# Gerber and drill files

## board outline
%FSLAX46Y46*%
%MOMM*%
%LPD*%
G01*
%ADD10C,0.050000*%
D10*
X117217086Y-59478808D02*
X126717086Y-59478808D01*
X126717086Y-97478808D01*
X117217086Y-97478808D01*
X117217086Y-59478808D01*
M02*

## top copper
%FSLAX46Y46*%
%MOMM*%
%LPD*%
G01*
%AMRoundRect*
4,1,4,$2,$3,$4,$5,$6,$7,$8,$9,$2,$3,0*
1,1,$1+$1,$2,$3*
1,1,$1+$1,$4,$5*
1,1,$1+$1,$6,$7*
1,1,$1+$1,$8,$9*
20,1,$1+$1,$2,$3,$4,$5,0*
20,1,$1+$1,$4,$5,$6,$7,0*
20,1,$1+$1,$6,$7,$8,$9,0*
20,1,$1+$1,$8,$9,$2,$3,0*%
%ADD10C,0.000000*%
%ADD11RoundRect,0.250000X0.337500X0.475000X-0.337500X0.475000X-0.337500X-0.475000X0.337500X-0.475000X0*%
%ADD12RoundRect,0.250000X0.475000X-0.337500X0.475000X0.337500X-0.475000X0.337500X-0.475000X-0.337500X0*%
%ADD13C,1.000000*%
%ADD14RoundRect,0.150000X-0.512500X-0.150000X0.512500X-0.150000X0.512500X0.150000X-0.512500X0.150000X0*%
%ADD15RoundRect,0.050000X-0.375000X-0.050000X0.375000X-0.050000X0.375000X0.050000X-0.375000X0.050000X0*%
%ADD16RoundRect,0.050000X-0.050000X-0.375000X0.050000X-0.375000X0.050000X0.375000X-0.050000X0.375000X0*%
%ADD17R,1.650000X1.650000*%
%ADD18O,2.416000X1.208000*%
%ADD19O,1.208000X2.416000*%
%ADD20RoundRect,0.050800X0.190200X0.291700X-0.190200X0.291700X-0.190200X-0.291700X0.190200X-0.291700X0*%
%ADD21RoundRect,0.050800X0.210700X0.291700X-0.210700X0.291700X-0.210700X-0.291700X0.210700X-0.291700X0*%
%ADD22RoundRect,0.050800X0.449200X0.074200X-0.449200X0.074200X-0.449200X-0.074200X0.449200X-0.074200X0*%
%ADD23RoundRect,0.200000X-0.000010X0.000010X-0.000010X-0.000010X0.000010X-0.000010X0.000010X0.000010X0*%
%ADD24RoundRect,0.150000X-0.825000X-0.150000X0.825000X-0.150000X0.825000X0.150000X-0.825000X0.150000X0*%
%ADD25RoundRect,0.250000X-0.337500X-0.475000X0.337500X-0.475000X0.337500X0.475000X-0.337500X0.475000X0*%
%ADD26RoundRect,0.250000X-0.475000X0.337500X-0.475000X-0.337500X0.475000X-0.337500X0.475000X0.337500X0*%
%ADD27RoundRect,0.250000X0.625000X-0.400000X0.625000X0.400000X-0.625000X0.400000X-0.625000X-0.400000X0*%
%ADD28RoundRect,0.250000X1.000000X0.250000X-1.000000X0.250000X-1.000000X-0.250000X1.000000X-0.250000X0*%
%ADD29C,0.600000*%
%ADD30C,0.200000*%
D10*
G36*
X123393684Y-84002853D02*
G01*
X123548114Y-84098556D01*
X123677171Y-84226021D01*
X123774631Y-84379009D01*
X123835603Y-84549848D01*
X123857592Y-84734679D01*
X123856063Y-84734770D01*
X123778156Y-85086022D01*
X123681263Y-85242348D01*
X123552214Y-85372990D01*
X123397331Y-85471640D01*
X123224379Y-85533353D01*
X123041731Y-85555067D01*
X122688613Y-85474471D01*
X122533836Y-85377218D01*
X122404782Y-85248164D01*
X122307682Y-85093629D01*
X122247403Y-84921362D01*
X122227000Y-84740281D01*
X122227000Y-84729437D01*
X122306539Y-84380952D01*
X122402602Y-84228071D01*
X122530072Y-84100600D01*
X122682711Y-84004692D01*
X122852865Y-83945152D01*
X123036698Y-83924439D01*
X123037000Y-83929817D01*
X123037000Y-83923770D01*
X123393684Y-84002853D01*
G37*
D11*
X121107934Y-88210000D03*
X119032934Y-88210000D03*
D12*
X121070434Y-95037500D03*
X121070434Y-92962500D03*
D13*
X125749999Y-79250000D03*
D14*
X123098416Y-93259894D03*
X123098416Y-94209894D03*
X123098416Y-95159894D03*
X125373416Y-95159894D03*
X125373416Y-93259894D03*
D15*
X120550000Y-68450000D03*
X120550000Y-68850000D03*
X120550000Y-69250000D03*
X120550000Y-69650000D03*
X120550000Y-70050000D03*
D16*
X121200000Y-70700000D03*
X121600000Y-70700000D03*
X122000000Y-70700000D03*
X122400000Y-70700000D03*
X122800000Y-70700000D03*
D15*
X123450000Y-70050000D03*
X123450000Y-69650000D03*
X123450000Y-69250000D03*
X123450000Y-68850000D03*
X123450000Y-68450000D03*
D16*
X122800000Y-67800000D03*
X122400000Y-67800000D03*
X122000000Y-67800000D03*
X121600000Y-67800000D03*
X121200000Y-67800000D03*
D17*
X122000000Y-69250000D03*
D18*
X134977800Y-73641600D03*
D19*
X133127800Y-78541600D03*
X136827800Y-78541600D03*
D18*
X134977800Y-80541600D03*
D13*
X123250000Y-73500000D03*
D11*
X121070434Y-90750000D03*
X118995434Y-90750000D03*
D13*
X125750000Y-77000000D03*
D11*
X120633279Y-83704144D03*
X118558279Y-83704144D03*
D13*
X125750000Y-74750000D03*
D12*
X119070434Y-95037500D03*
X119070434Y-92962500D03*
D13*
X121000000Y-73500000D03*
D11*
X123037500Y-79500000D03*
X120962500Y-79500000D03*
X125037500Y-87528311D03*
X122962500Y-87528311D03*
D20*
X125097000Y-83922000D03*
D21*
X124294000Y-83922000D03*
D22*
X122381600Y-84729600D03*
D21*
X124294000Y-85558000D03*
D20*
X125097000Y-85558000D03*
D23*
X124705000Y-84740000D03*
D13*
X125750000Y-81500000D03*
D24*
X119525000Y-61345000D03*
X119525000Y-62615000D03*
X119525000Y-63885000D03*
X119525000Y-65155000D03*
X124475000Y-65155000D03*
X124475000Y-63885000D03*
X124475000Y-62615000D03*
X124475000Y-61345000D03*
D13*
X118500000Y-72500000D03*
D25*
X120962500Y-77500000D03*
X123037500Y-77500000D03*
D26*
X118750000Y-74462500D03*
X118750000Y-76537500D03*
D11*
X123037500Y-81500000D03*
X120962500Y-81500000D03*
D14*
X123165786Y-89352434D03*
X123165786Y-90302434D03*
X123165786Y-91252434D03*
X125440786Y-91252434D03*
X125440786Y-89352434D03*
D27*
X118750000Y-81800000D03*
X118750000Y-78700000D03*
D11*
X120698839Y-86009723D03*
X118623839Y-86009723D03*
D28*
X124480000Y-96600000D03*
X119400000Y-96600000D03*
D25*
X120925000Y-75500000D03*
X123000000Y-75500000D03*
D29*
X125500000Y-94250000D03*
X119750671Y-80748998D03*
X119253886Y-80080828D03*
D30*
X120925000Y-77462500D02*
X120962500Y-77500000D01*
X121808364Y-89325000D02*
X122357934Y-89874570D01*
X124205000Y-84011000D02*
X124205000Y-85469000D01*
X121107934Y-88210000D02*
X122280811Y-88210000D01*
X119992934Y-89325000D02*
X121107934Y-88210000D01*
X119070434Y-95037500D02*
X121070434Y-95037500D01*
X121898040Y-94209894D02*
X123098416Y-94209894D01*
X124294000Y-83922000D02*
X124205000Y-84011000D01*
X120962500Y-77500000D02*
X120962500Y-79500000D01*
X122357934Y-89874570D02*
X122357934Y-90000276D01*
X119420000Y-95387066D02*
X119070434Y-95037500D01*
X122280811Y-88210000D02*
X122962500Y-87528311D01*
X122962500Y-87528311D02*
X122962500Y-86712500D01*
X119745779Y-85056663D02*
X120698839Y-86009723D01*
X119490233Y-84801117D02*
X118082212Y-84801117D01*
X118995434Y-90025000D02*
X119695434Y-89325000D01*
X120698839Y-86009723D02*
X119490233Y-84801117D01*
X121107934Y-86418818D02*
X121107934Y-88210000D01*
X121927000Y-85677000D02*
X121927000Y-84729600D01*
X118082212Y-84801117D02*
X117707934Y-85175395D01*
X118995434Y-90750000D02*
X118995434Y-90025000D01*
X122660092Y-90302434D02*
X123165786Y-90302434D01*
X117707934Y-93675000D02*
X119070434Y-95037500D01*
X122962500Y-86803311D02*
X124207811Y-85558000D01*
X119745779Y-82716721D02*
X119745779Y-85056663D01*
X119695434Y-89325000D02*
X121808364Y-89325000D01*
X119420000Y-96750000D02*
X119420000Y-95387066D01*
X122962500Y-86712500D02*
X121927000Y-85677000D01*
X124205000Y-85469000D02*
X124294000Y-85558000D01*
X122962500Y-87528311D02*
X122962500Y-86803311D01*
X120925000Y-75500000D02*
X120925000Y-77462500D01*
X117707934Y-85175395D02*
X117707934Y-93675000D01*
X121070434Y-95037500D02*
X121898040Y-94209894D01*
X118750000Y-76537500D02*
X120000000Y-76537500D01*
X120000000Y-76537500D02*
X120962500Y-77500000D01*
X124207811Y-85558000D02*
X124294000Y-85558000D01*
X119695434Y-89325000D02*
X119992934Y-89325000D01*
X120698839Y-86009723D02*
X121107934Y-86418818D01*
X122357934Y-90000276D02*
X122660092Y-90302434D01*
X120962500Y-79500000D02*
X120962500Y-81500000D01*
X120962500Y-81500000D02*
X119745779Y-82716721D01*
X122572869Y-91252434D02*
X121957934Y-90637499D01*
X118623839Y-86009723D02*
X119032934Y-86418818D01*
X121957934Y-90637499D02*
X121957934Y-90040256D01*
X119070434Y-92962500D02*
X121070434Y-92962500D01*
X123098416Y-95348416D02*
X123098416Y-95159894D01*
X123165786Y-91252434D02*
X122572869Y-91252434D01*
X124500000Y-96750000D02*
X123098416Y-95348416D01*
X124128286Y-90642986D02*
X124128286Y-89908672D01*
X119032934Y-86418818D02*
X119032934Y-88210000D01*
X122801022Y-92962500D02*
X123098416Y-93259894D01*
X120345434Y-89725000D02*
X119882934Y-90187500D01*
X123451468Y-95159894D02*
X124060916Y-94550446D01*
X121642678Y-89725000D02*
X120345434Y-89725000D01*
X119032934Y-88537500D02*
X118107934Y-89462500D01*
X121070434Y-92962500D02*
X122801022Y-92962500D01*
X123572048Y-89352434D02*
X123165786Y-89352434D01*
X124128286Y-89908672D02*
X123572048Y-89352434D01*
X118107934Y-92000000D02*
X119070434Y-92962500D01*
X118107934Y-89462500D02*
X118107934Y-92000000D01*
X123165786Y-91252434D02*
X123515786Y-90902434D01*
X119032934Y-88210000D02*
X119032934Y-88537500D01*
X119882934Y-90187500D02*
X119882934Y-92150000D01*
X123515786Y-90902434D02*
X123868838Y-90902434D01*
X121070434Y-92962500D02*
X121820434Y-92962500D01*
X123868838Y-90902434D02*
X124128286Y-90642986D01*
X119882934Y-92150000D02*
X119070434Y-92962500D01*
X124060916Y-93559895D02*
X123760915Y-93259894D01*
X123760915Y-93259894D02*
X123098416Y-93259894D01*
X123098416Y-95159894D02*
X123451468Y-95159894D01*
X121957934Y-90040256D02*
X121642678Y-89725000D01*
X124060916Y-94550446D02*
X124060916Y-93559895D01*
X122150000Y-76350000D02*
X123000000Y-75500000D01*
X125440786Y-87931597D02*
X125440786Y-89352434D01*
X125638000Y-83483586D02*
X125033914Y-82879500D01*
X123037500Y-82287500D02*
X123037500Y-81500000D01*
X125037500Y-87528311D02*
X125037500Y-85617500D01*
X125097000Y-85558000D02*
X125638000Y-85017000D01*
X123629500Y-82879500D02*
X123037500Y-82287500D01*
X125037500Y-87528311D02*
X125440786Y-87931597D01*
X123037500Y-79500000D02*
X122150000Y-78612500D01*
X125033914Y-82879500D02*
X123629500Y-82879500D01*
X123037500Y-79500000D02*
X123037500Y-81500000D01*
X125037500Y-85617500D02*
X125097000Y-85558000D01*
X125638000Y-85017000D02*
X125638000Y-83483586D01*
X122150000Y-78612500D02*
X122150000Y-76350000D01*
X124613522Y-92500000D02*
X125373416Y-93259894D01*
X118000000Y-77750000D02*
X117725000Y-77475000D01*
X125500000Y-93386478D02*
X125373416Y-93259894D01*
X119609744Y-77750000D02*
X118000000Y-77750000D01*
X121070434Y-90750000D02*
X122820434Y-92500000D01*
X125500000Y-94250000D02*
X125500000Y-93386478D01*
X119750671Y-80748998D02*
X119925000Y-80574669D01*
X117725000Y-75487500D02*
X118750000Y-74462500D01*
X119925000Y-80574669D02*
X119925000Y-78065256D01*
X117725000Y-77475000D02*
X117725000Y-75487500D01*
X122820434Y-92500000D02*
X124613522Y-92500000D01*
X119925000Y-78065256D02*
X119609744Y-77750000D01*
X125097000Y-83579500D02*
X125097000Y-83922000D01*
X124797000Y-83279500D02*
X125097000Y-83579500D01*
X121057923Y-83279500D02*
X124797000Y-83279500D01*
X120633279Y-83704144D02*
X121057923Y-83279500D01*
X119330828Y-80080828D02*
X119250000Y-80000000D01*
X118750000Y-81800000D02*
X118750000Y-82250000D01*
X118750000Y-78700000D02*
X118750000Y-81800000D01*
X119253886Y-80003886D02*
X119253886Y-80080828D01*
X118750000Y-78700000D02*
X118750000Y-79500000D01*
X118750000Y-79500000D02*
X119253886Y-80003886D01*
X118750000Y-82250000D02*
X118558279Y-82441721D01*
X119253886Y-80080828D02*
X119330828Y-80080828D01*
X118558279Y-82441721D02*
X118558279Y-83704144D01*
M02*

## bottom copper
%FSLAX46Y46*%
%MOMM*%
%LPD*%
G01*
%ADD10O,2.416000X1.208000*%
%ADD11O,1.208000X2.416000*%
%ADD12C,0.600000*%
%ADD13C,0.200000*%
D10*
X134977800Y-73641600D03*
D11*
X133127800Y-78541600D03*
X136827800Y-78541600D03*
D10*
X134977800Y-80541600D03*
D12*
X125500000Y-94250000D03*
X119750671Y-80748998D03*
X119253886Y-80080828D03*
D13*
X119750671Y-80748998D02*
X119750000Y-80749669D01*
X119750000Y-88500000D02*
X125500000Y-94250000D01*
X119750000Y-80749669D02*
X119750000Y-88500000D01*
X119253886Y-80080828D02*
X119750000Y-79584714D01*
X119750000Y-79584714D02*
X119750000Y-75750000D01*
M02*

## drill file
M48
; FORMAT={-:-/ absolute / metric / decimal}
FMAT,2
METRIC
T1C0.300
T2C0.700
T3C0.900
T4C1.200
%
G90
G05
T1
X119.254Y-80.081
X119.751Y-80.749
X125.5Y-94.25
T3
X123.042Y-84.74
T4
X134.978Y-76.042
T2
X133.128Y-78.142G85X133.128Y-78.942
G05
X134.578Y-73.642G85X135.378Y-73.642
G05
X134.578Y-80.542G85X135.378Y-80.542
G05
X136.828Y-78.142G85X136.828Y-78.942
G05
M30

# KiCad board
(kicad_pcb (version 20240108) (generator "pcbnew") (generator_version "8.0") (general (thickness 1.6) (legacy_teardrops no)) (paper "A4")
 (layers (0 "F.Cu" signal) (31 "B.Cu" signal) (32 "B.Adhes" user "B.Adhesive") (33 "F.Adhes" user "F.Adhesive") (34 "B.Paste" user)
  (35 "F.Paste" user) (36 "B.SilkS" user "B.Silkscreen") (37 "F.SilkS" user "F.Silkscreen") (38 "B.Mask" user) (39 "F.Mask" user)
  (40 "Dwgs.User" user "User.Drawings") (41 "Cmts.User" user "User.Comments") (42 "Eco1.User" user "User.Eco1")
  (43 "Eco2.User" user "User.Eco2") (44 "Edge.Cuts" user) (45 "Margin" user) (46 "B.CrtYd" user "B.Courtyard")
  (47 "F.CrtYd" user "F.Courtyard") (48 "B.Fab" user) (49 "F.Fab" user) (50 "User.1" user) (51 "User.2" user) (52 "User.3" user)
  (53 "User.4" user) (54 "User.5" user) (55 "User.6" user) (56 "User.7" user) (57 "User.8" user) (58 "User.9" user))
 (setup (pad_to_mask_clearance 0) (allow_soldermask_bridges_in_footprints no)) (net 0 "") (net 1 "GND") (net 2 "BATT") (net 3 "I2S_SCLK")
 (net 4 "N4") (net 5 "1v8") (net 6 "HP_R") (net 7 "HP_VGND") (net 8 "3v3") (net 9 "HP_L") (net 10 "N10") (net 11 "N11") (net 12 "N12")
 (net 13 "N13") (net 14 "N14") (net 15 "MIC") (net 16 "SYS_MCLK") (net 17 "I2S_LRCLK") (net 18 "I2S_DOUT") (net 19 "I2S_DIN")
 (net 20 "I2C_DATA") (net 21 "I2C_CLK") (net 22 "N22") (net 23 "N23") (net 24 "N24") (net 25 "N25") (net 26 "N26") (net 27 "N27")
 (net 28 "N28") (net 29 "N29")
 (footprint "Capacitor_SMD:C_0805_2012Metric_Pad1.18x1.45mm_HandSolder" (layer "F.Cu") (at 120.070434 88.21 180)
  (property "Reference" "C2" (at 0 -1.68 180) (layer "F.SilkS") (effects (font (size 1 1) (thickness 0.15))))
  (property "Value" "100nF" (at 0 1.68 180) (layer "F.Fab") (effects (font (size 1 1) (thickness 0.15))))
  (pad "1" smd roundrect (at -1.0375 0 180) (size 1.175 1.45) (layers "F.Cu" "F.Paste" "F.Mask") (roundrect_rratio 0.212766) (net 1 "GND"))
  (pad "2" smd roundrect (at 1.0375 0 180) (size 1.175 1.45) (layers "F.Cu" "F.Paste" "F.Mask") (roundrect_rratio 0.212766) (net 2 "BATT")))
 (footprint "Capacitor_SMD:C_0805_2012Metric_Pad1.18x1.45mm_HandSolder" (layer "F.Cu") (at 121.070434 94 90)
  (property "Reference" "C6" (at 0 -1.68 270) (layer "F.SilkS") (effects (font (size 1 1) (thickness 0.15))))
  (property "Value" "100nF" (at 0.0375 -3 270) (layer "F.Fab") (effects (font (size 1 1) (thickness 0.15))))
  (pad "1" smd roundrect (at -1.0375 0 90) (size 1.175 1.45) (layers "F.Cu" "F.Paste" "F.Mask") (roundrect_rratio 0.212766) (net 1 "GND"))
  (pad "2" smd roundrect (at 1.0375 0 90) (size 1.175 1.45) (layers "F.Cu" "F.Paste" "F.Mask") (roundrect_rratio 0.212766) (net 2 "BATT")))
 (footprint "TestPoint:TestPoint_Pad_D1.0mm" (layer "F.Cu") (at 125.749999 79.25)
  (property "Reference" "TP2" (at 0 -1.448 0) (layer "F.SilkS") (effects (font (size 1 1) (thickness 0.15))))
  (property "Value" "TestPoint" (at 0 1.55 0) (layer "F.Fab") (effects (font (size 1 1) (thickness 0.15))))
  (pad "1" smd circle (at 0 0) (size 1 1) (layers "F.Cu" "F.Mask") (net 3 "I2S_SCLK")))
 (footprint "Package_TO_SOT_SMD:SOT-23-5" (layer "F.Cu") (at 124.235916 94.209894)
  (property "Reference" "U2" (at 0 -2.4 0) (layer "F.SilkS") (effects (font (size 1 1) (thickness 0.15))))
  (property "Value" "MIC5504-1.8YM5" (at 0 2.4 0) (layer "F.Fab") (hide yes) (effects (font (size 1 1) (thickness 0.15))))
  (pad "1" smd roundrect (at -1.1375 -0.95) (size 1.325 0.6) (layers "F.Cu" "F.Paste" "F.Mask") (roundrect_rratio 0.25) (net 2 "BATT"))
  (pad "2" smd roundrect (at -1.1375 0) (size 1.325 0.6) (layers "F.Cu" "F.Paste" "F.Mask") (roundrect_rratio 0.25) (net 1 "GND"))
  (pad "3" smd roundrect (at -1.1375 0.95) (size 1.325 0.6) (layers "F.Cu" "F.Paste" "F.Mask") (roundrect_rratio 0.25) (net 2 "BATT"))
  (pad "4" smd roundrect (at 1.1375 0.95) (size 1.325 0.6) (layers "F.Cu" "F.Paste" "F.Mask") (roundrect_rratio 0.25) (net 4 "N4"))
  (pad "5" smd roundrect (at 1.1375 -0.95) (size 1.325 0.6) (layers "F.Cu" "F.Paste" "F.Mask") (roundrect_rratio 0.25) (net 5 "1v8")))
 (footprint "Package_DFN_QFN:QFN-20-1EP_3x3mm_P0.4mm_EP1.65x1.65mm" (layer "F.Cu") (at 122 69.25)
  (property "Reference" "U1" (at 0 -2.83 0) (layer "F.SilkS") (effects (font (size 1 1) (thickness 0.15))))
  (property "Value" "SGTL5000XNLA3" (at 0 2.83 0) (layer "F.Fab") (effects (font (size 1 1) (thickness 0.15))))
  (pad "" smd roundrect (at -0.41 -0.41) (size 0.67 0.67) (layers "F.Paste") (roundrect_rratio 0.25))
  (pad "" smd roundrect (at -0.41 0.41) (size 0.67 0.67) (layers "F.Paste") (roundrect_rratio 0.25))
  (pad "" smd roundrect (at 0.41 -0.41) (size 0.67 0.67) (layers "F.Paste") (roundrect_rratio 0.25))
  (pad "" smd roundrect (at 0.41 0.41) (size 0.67 0.67) (layers "F.Paste") (roundrect_rratio 0.25))
  (pad "1" smd roundrect (at -1.45 -0.8) (size 0.85 0.2) (layers "F.Cu" "F.Paste" "F.Mask") (roundrect_rratio 0.25) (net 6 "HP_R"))
  (pad "2" smd roundrect (at -1.45 -0.4) (size 0.85 0.2) (layers "F.Cu" "F.Paste" "F.Mask") (roundrect_rratio 0.25) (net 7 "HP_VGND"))
  (pad "3" smd roundrect (at -1.45 0) (size 0.85 0.2) (layers "F.Cu" "F.Paste" "F.Mask") (roundrect_rratio 0.25) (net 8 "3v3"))
  (pad "4" smd roundrect (at -1.45 0.4) (size 0.85 0.2) (layers "F.Cu" "F.Paste" "F.Mask") (roundrect_rratio 0.25) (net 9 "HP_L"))
  (pad "5" smd roundrect (at -1.45 0.8) (size 0.85 0.2) (layers "F.Cu" "F.Paste" "F.Mask") (roundrect_rratio 0.25) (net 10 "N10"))
  (pad "6" smd roundrect (at -0.8 1.45) (size 0.2 0.85) (layers "F.Cu" "F.Paste" "F.Mask") (roundrect_rratio 0.25) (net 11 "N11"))
  (pad "7" smd roundrect (at -0.4 1.45) (size 0.2 0.85) (layers "F.Cu" "F.Paste" "F.Mask") (roundrect_rratio 0.25) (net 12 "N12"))
  (pad "8" smd roundrect (at 0 1.45) (size 0.2 0.85) (layers "F.Cu" "F.Paste" "F.Mask") (roundrect_rratio 0.25) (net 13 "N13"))
  (pad "9" smd roundrect (at 0.4 1.45) (size 0.2 0.85) (layers "F.Cu" "F.Paste" "F.Mask") (roundrect_rratio 0.25) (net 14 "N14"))
  (pad "10" smd roundrect (at 0.8 1.45) (size 0.2 0.85) (layers "F.Cu" "F.Paste" "F.Mask") (roundrect_rratio 0.25) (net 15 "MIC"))
  (pad "11" smd roundrect (at 1.45 0.8) (size 0.85 0.2) (layers "F.Cu" "F.Paste" "F.Mask") (roundrect_rratio 0.25) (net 15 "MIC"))
  (pad "12" smd roundrect (at 1.45 0.4) (size 0.85 0.2) (layers "F.Cu" "F.Paste" "F.Mask") (roundrect_rratio 0.25) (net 8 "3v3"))
  (pad "13" smd roundrect (at 1.45 0) (size 0.85 0.2) (layers "F.Cu" "F.Paste" "F.Mask") (roundrect_rratio 0.25) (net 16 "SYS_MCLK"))
  (pad "14" smd roundrect (at 1.45 -0.4) (size 0.85 0.2) (layers "F.Cu" "F.Paste" "F.Mask") (roundrect_rratio 0.25) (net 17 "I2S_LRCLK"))
  (pad "15" smd roundrect (at 1.45 -0.8) (size 0.85 0.2) (layers "F.Cu" "F.Paste" "F.Mask") (roundrect_rratio 0.25) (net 3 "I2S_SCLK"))
  (pad "16" smd roundrect (at 0.8 -1.45) (size 0.2 0.85) (layers "F.Cu" "F.Paste" "F.Mask") (roundrect_rratio 0.25) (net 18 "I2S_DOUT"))
  (pad "17" smd roundrect (at 0.4 -1.45) (size 0.2 0.85) (layers "F.Cu" "F.Paste" "F.Mask") (roundrect_rratio 0.25) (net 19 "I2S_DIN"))
  (pad "18" smd roundrect (at 0 -1.45) (size 0.2 0.85) (layers "F.Cu" "F.Paste" "F.Mask") (roundrect_rratio 0.25) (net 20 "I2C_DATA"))
  (pad "19" smd roundrect (at -0.4 -1.45) (size 0.2 0.85) (layers "F.Cu" "F.Paste" "F.Mask") (roundrect_rratio 0.25) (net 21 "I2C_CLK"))
  (pad "20" smd roundrect (at -0.8 -1.45) (size 0.2 0.85) (layers "F.Cu" "F.Paste" "F.Mask") (roundrect_rratio 0.25) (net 5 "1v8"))
  (pad "21" smd rect (at 0 0) (size 1.65 1.65) (layers "F.Cu" "F.Mask") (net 1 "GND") (zone_connect 2)))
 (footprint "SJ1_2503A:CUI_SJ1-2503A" (layer "F.Cu") (at 134.9778 73.6416)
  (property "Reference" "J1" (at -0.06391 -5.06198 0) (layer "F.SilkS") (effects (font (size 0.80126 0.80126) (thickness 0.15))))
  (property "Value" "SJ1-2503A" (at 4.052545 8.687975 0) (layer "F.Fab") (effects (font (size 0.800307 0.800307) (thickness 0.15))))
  (pad "" np_thru_hole circle (at 0 2.4) (size 1.2 1.2) (drill 1.2) (layers "*.Cu" "*.Mask"))
  (pad "1" thru_hole oval (at 0 0) (size 2.416 1.208) (drill oval 1.5 0.7) (layers "*.Cu" "*.Mask") (remove_unused_layers no)
   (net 7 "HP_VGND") (solder_mask_margin 0.102))
  (pad "2" thru_hole oval (at -1.85 4.9) (size 1.208 2.416) (drill oval 0.7 1.5) (layers "*.Cu" "*.Mask") (remove_unused_layers no)
   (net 6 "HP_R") (solder_mask_margin 0.102))
  (pad "3" thru_hole oval (at 1.85 4.9) (size 1.208 2.416) (drill oval 0.7 1.5) (layers "*.Cu" "*.Mask") (remove_unused_layers no)
   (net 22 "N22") (solder_mask_margin 0.102))
  (pad "4" thru_hole oval (at 0 6.9) (size 2.416 1.208) (drill oval 1.5 0.7) (layers "*.Cu" "*.Mask") (remove_unused_layers no)
   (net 9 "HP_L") (solder_mask_margin 0.102)))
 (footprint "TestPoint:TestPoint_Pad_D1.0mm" (layer "F.Cu") (at 123.25 73.5)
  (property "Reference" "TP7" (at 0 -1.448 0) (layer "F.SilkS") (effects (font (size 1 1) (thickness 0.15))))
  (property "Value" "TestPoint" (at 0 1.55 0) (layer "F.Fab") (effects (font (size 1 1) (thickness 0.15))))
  (pad "1" smd circle (at 0 0) (size 1 1) (layers "F.Cu" "F.Mask") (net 16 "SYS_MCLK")))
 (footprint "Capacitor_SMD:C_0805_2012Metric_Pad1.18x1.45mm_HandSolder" (layer "F.Cu") (at 120.032934 90.75 180)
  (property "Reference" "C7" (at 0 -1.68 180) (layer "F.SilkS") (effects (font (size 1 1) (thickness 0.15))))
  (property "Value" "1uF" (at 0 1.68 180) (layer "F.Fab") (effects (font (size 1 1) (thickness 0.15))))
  (pad "1" smd roundrect (at -1.0375 0 180) (size 1.175 1.45) (layers "F.Cu" "F.Paste" "F.Mask") (roundrect_rratio 0.212766) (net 5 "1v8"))
  (pad "2" smd roundrect (at 1.0375 0 180) (size 1.175 1.45) (layers "F.Cu" "F.Paste" "F.Mask") (roundrect_rratio 0.212766) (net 1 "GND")))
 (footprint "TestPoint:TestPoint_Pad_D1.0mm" (layer "F.Cu") (at 125.75 77)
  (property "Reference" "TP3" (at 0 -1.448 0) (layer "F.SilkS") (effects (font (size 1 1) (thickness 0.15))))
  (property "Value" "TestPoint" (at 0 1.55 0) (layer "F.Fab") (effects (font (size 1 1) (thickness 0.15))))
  (pad "1" smd circle (at 0 0) (size 1 1) (layers "F.Cu" "F.Mask") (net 18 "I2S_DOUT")))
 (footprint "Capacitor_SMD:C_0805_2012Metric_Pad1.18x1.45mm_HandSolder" (layer "F.Cu") (at 119.595779 83.704144 180)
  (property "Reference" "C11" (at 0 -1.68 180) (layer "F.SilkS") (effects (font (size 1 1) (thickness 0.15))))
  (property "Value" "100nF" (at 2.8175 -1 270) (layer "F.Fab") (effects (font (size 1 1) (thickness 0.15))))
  (pad "1" smd roundrect (at -1.0375 0 180) (size 1.175 1.45) (layers "F.Cu" "F.Paste" "F.Mask") (roundrect_rratio 0.212766) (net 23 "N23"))
  (pad "2" smd roundrect (at 1.0375 0 180) (size 1.175 1.45) (layers "F.Cu" "F.Paste" "F.Mask") (roundrect_rratio 0.212766) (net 15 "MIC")))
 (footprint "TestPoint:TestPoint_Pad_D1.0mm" (layer "F.Cu") (at 125.75 74.75)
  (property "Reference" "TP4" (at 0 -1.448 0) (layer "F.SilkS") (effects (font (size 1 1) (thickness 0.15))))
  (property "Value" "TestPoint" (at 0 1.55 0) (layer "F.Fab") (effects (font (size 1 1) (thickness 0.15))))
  (pad "1" smd circle (at 0 0) (size 1 1) (layers "F.Cu" "F.Mask") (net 19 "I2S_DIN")))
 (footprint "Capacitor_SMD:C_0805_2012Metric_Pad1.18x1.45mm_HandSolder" (layer "F.Cu") (at 119.070434 94 90)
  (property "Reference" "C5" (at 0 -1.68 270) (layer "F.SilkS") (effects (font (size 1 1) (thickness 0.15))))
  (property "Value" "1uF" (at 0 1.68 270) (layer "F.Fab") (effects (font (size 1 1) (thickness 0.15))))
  (pad "1" smd roundrect (at -1.0375 0 90) (size 1.175 1.45) (layers "F.Cu" "F.Paste" "F.Mask") (roundrect_rratio 0.212766) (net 1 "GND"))
  (pad "2" smd roundrect (at 1.0375 0 90) (size 1.175 1.45) (layers "F.Cu" "F.Paste" "F.Mask") (roundrect_rratio 0.212766) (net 2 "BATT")))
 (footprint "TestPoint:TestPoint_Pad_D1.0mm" (layer "F.Cu") (at 121 73.5)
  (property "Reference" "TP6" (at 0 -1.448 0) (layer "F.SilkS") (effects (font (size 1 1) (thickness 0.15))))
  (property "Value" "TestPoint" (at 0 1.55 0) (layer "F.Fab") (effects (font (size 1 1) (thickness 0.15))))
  (pad "1" smd circle (at 0 0) (size 1 1) (layers "F.Cu" "F.Mask") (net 21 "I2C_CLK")))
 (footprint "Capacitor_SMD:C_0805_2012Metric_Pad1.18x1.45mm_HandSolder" (layer "F.Cu") (at 122 79.5 180)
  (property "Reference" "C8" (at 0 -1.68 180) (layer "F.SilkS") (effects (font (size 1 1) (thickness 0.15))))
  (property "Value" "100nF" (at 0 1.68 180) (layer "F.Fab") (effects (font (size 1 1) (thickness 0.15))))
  (pad "1" smd roundrect (at -1.0375 0 180) (size 1.175 1.45) (layers "F.Cu" "F.Paste" "F.Mask") (roundrect_rratio 0.212766) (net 8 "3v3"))
  (pad "2" smd roundrect (at 1.0375 0 180) (size 1.175 1.45) (layers "F.Cu" "F.Paste" "F.Mask") (roundrect_rratio 0.212766) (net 1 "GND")))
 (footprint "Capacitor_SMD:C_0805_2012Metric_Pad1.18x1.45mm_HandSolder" (layer "F.Cu") (at 124 87.528311 180)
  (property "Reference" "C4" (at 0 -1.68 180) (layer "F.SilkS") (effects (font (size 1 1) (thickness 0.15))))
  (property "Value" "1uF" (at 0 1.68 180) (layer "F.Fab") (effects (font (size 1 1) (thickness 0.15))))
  (pad "1" smd roundrect (at -1.0375 0 180) (size 1.175 1.45) (layers "F.Cu" "F.Paste" "F.Mask") (roundrect_rratio 0.212766) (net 8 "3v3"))
  (pad "2" smd roundrect (at 1.0375 0 180) (size 1.175 1.45) (layers "F.Cu" "F.Paste" "F.Mask") (roundrect_rratio 0.212766) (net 1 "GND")))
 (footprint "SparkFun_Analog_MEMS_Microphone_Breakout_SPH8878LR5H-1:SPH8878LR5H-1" (layer "F.Cu") (at 123.042 84.74 -90)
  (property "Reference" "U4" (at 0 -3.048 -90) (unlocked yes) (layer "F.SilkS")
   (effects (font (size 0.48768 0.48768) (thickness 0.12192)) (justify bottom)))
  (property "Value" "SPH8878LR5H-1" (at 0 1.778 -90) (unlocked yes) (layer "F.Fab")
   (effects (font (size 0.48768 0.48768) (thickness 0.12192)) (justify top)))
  (fp_poly
   (pts (xy -0.00523 -0.814063) (xy 0.346022 -0.736156) (xy 0.502348 -0.639263) (xy 0.63299 -0.510214) (xy 0.73164 -0.355331)
    (xy 0.793353 -0.182379) (xy 0.815067 0.000269) (xy 0.734471 0.353387) (xy 0.637218 0.508164) (xy 0.508164 0.637218)
    (xy 0.353629 0.734318) (xy 0.181362 0.794597) (xy 0.000281 0.815) (xy -0.010563 0.815) (xy -0.359048 0.735461) (xy -0.511929 0.639398)
    (xy -0.6394 0.511928) (xy -0.735308 0.359289) (xy -0.794848 0.189135) (xy -0.815561 0.005302) (xy -0.810183 0.005) (xy -0.81623 0.005)
    (xy -0.737147 -0.351684) (xy -0.641444 -0.506114) (xy -0.513979 -0.635171) (xy -0.360991 -0.732631) (xy -0.190152 -0.793603)
    (xy -0.005321 -0.815592))
   (stroke (width 0) (type default)) (fill solid) (layer "F.Cu"))
  (pad "" np_thru_hole circle (at 0 0 270) (size 0.9 0.9) (drill 0.9) (layers "*.Cu" "*.Mask"))
  (pad "1" smd roundrect (at -0.818 -2.055 180) (size 0.482 0.685) (layers "F.Cu" "F.Paste" "F.Mask") (roundrect_rratio 0.1053941909)
   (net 23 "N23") (solder_mask_margin 0.0635) (thermal_bridge_angle 0))
  (pad "2" smd roundrect (at -0.818 -1.252 180) (size 0.523 0.685) (layers "F.Cu" "F.Paste" "F.Mask") (roundrect_rratio 0.09713193117)
   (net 1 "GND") (solder_mask_margin 0.0635) (thermal_bridge_angle 0))
  (pad "3" smd roundrect (at -0.0104 0.6604 180) (size 1 0.25) (layers "F.Cu") (roundrect_rratio 0.2032) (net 1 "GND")
   (solder_mask_margin 0.0635) (thermal_bridge_angle 0))
  (pad "4" smd roundrect (at 0.818 -1.252 180) (size 0.523 0.685) (layers "F.Cu" "F.Paste" "F.Mask") (roundrect_rratio 0.09713193117)
   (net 1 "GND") (solder_mask_margin 0.0635) (thermal_bridge_angle 0))
  (pad "5" smd roundrect (at 0.818 -2.055 180) (size 0.482 0.685) (layers "F.Cu" "F.Paste" "F.Mask") (roundrect_rratio 0.1053941909)
   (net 8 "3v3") (solder_mask_margin 0.0635) (thermal_bridge_angle 0))
  (pad "6" smd roundrect (at 0 -1.663 270) (size 0.4 0.4) (layers "F.Cu" "F.Paste" "F.Mask") (roundrect_rratio 0.5) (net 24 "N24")
   (solder_mask_margin 0.0635) (thermal_bridge_angle 0)))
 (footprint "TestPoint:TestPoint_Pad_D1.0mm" (layer "F.Cu") (at 125.75 81.5)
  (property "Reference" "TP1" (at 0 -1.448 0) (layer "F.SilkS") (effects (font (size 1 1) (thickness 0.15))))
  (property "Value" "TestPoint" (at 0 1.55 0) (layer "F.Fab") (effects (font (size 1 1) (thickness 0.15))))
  (pad "1" smd circle (at 0 0) (size 1 1) (layers "F.Cu" "F.Mask") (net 17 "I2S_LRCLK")))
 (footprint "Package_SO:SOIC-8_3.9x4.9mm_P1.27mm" (layer "F.Cu") (at 122 63.25)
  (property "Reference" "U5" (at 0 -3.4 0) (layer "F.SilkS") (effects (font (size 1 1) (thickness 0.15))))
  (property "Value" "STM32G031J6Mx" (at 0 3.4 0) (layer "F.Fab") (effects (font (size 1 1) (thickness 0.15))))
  (pad "1" smd roundrect (at -2.475 -1.905) (size 1.95 0.6) (layers "F.Cu" "F.Paste" "F.Mask") (roundrect_rratio 0.25) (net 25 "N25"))
  (pad "2" smd roundrect (at -2.475 -0.635) (size 1.95 0.6) (layers "F.Cu" "F.Paste" "F.Mask") (roundrect_rratio 0.25) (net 8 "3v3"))
  (pad "3" smd roundrect (at -2.475 0.635) (size 1.95 0.6) (layers "F.Cu" "F.Paste" "F.Mask") (roundrect_rratio 0.25) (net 1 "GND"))
  (pad "4" smd roundrect (at -2.475 1.905) (size 1.95 0.6) (layers "F.Cu" "F.Paste" "F.Mask") (roundrect_rratio 0.25) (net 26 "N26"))
  (pad "5" smd roundrect (at 2.475 1.905) (size 1.95 0.6) (layers "F.Cu" "F.Paste" "F.Mask") (roundrect_rratio 0.25) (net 21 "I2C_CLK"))
  (pad "6" smd roundrect (at 2.475 0.635) (size 1.95 0.6) (layers "F.Cu" "F.Paste" "F.Mask") (roundrect_rratio 0.25) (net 20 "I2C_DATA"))
  (pad "7" smd roundrect (at 2.475 -0.635) (size 1.95 0.6) (layers "F.Cu" "F.Paste" "F.Mask") (roundrect_rratio 0.25) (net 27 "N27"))
  (pad "8" smd roundrect (at 2.475 -1.905) (size 1.95 0.6) (layers "F.Cu" "F.Paste" "F.Mask") (roundrect_rratio 0.25) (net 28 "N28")))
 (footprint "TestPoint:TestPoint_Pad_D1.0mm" (layer "F.Cu") (at 118.5 72.5)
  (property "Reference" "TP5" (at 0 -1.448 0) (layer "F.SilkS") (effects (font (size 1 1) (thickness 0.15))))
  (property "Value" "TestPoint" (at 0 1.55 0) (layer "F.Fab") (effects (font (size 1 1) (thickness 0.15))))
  (pad "1" smd circle (at 0 0) (size 1 1) (layers "F.Cu" "F.Mask") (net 20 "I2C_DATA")))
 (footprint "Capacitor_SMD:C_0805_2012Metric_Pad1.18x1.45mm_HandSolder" (layer "F.Cu") (at 122 77.5)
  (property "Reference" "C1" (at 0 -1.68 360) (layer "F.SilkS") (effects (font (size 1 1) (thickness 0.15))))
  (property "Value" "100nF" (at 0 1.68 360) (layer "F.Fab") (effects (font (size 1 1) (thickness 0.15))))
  (pad "1" smd roundrect (at -1.0375 0) (size 1.175 1.45) (layers "F.Cu" "F.Paste" "F.Mask") (roundrect_rratio 0.212766) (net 1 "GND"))
  (pad "2" smd roundrect (at 1.0375 0) (size 1.175 1.45) (layers "F.Cu" "F.Paste" "F.Mask") (roundrect_rratio 0.212766) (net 10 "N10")))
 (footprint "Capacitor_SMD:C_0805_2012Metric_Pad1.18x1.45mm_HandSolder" (layer "F.Cu") (at 118.75 75.5 -90)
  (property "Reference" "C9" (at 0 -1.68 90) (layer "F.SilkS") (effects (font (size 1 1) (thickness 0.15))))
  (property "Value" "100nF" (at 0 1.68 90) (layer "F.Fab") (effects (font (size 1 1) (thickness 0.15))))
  (pad "1" smd roundrect (at -1.0375 0 270) (size 1.175 1.45) (layers "F.Cu" "F.Paste" "F.Mask") (roundrect_rratio 0.212766) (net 5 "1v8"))
  (pad "2" smd roundrect (at 1.0375 0 270) (size 1.175 1.45) (layers "F.Cu" "F.Paste" "F.Mask") (roundrect_rratio 0.212766) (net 1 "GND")))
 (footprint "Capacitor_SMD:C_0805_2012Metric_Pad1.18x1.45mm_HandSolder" (layer "F.Cu") (at 122 81.5 180)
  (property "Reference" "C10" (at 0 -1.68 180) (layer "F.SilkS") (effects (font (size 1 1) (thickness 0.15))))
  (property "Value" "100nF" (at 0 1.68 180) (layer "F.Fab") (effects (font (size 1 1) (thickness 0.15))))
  (pad "1" smd roundrect (at -1.0375 0 180) (size 1.175 1.45) (layers "F.Cu" "F.Paste" "F.Mask") (roundrect_rratio 0.212766) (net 8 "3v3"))
  (pad "2" smd roundrect (at 1.0375 0 180) (size 1.175 1.45) (layers "F.Cu" "F.Paste" "F.Mask") (roundrect_rratio 0.212766) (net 1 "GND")))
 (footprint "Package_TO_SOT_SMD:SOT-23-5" (layer "F.Cu") (at 124.303286 90.302434)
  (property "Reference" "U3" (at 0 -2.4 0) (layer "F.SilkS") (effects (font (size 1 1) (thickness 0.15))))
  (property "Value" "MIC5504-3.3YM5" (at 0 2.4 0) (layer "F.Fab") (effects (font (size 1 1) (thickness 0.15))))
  (pad "1" smd roundrect (at -1.1375 -0.95) (size 1.325 0.6) (layers "F.Cu" "F.Paste" "F.Mask") (roundrect_rratio 0.25) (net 2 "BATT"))
  (pad "2" smd roundrect (at -1.1375 0) (size 1.325 0.6) (layers "F.Cu" "F.Paste" "F.Mask") (roundrect_rratio 0.25) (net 1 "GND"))
  (pad "3" smd roundrect (at -1.1375 0.95) (size 1.325 0.6) (layers "F.Cu" "F.Paste" "F.Mask") (roundrect_rratio 0.25) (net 2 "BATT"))
  (pad "4" smd roundrect (at 1.1375 0.95) (size 1.325 0.6) (layers "F.Cu" "F.Paste" "F.Mask") (roundrect_rratio 0.25) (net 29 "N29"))
  (pad "5" smd roundrect (at 1.1375 -0.95) (size 1.325 0.6) (layers "F.Cu" "F.Paste" "F.Mask") (roundrect_rratio 0.25) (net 8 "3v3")))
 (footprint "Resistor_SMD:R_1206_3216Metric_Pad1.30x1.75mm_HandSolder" (layer "F.Cu") (at 118.75 80.25 90)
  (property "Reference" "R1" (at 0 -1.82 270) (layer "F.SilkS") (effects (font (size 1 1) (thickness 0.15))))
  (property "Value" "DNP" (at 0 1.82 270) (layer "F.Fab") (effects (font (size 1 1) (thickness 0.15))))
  (pad "1" smd roundrect (at -1.55 0 90) (size 1.3 1.75) (layers "F.Cu" "F.Paste" "F.Mask") (roundrect_rratio 0.192308) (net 15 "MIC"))
  (pad "2" smd roundrect (at 1.55 0 90) (size 1.3 1.75) (layers "F.Cu" "F.Paste" "F.Mask") (roundrect_rratio 0.192308) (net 15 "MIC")))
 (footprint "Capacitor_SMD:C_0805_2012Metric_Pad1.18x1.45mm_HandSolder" (layer "F.Cu") (at 119.661339 86.009723 180)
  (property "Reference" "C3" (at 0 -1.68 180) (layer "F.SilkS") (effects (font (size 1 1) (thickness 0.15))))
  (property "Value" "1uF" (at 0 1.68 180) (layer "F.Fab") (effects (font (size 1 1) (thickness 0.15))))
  (pad "1" smd roundrect (at -1.0375 0 180) (size 1.175 1.45) (layers "F.Cu" "F.Paste" "F.Mask") (roundrect_rratio 0.212766) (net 1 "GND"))
  (pad "2" smd roundrect (at 1.0375 0 180) (size 1.175 1.45) (layers "F.Cu" "F.Paste" "F.Mask") (roundrect_rratio 0.212766) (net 2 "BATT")))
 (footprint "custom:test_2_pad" (layer "F.Cu") (at 121.94 101.68 180)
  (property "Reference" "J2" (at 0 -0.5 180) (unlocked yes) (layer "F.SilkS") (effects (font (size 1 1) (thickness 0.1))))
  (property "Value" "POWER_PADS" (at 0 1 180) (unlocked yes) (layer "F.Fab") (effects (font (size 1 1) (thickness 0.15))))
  (pad "1" smd roundrect (at -2.54 5.08 180) (size 2.5 1) (layers "F.Cu" "F.Paste" "F.Mask") (roundrect_rratio 0.25) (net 2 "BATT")
   (thermal_bridge_angle 45))
  (pad "2" smd roundrect (at 2.54 5.08 180) (size 2.5 1) (layers "F.Cu" "F.Paste" "F.Mask") (roundrect_rratio 0.25) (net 1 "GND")
   (thermal_bridge_angle 45)))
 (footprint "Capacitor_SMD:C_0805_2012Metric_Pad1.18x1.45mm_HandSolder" (layer "F.Cu") (at 121.9625 75.5)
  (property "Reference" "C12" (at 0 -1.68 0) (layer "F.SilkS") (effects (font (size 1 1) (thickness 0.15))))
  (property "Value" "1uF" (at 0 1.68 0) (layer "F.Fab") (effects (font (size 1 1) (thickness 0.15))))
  (pad "1" smd roundrect (at -1.0375 0) (size 1.175 1.45) (layers "F.Cu" "F.Paste" "F.Mask") (roundrect_rratio 0.212766) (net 1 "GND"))
  (pad "2" smd roundrect (at 1.0375 0) (size 1.175 1.45) (layers "F.Cu" "F.Paste" "F.Mask") (roundrect_rratio 0.212766) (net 8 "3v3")))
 (gr_rect (start 117.217086 59.478808) (end 126.717086 97.478808) (stroke (width 0.05) (type default)) (fill none) (layer "Edge.Cuts"))
 (segment (start 120.925 77.4625) (end 120.9625 77.5) (width 0.2) (layer "F.Cu") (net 1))
 (segment (start 121.808364 89.325) (end 122.357934 89.87457) (width 0.2) (layer "F.Cu") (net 1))
 (segment (start 124.205 84.011) (end 124.205 85.469) (width 0.2) (layer "F.Cu") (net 1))
 (segment (start 121.107934 88.21) (end 122.280811 88.21) (width 0.2) (layer "F.Cu") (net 1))
 (segment (start 119.992934 89.325) (end 121.107934 88.21) (width 0.2) (layer "F.Cu") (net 1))
 (segment (start 119.070434 95.0375) (end 121.070434 95.0375) (width 0.2) (layer "F.Cu") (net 1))
 (segment (start 121.89804 94.209894) (end 123.098416 94.209894) (width 0.2) (layer "F.Cu") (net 1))
 (segment (start 124.294 83.922) (end 124.205 84.011) (width 0.2) (layer "F.Cu") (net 1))
 (segment (start 120.9625 77.5) (end 120.9625 79.5) (width 0.2) (layer "F.Cu") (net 1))
 (segment (start 122.357934 89.87457) (end 122.357934 90.000276) (width 0.2) (layer "F.Cu") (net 1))
 (segment (start 119.42 95.387066) (end 119.070434 95.0375) (width 0.2) (layer "F.Cu") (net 1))
 (segment (start 122.280811 88.21) (end 122.9625 87.528311) (width 0.2) (layer "F.Cu") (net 1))
 (segment (start 122.9625 87.528311) (end 122.9625 86.7125) (width 0.2) (layer "F.Cu") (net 1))
 (segment (start 119.745779 85.056663) (end 120.698839 86.009723) (width 0.2) (layer "F.Cu") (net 1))
 (segment (start 119.490233 84.801117) (end 118.082212 84.801117) (width 0.2) (layer "F.Cu") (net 1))
 (segment (start 118.995434 90.025) (end 119.695434 89.325) (width 0.2) (layer "F.Cu") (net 1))
 (segment (start 120.698839 86.009723) (end 119.490233 84.801117) (width 0.2) (layer "F.Cu") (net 1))
 (segment (start 121.107934 86.418818) (end 121.107934 88.21) (width 0.2) (layer "F.Cu") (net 1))
 (segment (start 121.927 85.677) (end 121.927 84.7296) (width 0.2) (layer "F.Cu") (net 1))
 (segment (start 118.082212 84.801117) (end 117.707934 85.175395) (width 0.2) (layer "F.Cu") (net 1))
 (segment (start 118.995434 90.75) (end 118.995434 90.025) (width 0.2) (layer "F.Cu") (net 1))
 (segment (start 122.660092 90.302434) (end 123.165786 90.302434) (width 0.2) (layer "F.Cu") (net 1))
 (segment (start 117.707934 93.675) (end 119.070434 95.0375) (width 0.2) (layer "F.Cu") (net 1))
 (segment (start 122.9625 86.803311) (end 124.207811 85.558) (width 0.2) (layer "F.Cu") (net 1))
 (segment (start 119.745779 82.716721) (end 119.745779 85.056663) (width 0.2) (layer "F.Cu") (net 1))
 (segment (start 119.695434 89.325) (end 121.808364 89.325) (width 0.2) (layer "F.Cu") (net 1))
 (segment (start 119.42 96.75) (end 119.42 95.387066) (width 0.2) (layer "F.Cu") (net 1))
 (segment (start 122.9625 86.7125) (end 121.927 85.677) (width 0.2) (layer "F.Cu") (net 1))
 (segment (start 124.205 85.469) (end 124.294 85.558) (width 0.2) (layer "F.Cu") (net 1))
 (segment (start 122.9625 87.528311) (end 122.9625 86.803311) (width 0.2) (layer "F.Cu") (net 1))
 (segment (start 120.925 75.5) (end 120.925 77.4625) (width 0.2) (layer "F.Cu") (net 1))
 (segment (start 117.707934 85.175395) (end 117.707934 93.675) (width 0.2) (layer "F.Cu") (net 1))
 (segment (start 121.070434 95.0375) (end 121.89804 94.209894) (width 0.2) (layer "F.Cu") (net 1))
 (segment (start 118.75 76.5375) (end 120 76.5375) (width 0.2) (layer "F.Cu") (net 1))
 (segment (start 120 76.5375) (end 120.9625 77.5) (width 0.2) (layer "F.Cu") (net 1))
 (segment (start 124.207811 85.558) (end 124.294 85.558) (width 0.2) (layer "F.Cu") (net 1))
 (segment (start 119.695434 89.325) (end 119.992934 89.325) (width 0.2) (layer "F.Cu") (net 1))
 (segment (start 120.698839 86.009723) (end 121.107934 86.418818) (width 0.2) (layer "F.Cu") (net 1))
 (segment (start 122.357934 90.000276) (end 122.660092 90.302434) (width 0.2) (layer "F.Cu") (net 1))
 (segment (start 120.9625 79.5) (end 120.9625 81.5) (width 0.2) (layer "F.Cu") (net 1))
 (segment (start 120.9625 81.5) (end 119.745779 82.716721) (width 0.2) (layer "F.Cu") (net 1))
 (segment (start 122.572869 91.252434) (end 121.957934 90.637499) (width 0.2) (layer "F.Cu") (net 2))
 (segment (start 118.623839 86.009723) (end 119.032934 86.418818) (width 0.2) (layer "F.Cu") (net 2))
 (segment (start 121.957934 90.637499) (end 121.957934 90.040256) (width 0.2) (layer "F.Cu") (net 2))
 (segment (start 119.070434 92.9625) (end 121.070434 92.9625) (width 0.2) (layer "F.Cu") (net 2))
 (segment (start 123.098416 95.348416) (end 123.098416 95.159894) (width 0.2) (layer "F.Cu") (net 2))
 (segment (start 123.165786 91.252434) (end 122.572869 91.252434) (width 0.2) (layer "F.Cu") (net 2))
 (segment (start 124.5 96.75) (end 123.098416 95.348416) (width 0.2) (layer "F.Cu") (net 2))
 (segment (start 124.128286 90.642986) (end 124.128286 89.908672) (width 0.2) (layer "F.Cu") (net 2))
 (segment (start 119.032934 86.418818) (end 119.032934 88.21) (width 0.2) (layer "F.Cu") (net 2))
 (segment (start 122.801022 92.9625) (end 123.098416 93.259894) (width 0.2) (layer "F.Cu") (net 2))
 (segment (start 120.345434 89.725) (end 119.882934 90.1875) (width 0.2) (layer "F.Cu") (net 2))
 (segment (start 123.451468 95.159894) (end 124.060916 94.550446) (width 0.2) (layer "F.Cu") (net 2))
 (segment (start 121.642678 89.725) (end 120.345434 89.725) (width 0.2) (layer "F.Cu") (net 2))
 (segment (start 119.032934 88.5375) (end 118.107934 89.4625) (width 0.2) (layer "F.Cu") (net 2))
 (segment (start 121.070434 92.9625) (end 122.801022 92.9625) (width 0.2) (layer "F.Cu") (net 2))
 (segment (start 123.572048 89.352434) (end 123.165786 89.352434) (width 0.2) (layer "F.Cu") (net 2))
 (segment (start 124.128286 89.908672) (end 123.572048 89.352434) (width 0.2) (layer "F.Cu") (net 2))
 (segment (start 118.107934 92) (end 119.070434 92.9625) (width 0.2) (layer "F.Cu") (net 2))
 (segment (start 118.107934 89.4625) (end 118.107934 92) (width 0.2) (layer "F.Cu") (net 2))
 (segment (start 123.165786 91.252434) (end 123.515786 90.902434) (width 0.2) (layer "F.Cu") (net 2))
 (segment (start 119.032934 88.21) (end 119.032934 88.5375) (width 0.2) (layer "F.Cu") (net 2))
 (segment (start 119.882934 90.1875) (end 119.882934 92.15) (width 0.2) (layer "F.Cu") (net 2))
 (segment (start 123.515786 90.902434) (end 123.868838 90.902434) (width 0.2) (layer "F.Cu") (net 2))
 (segment (start 121.070434 92.9625) (end 121.820434 92.9625) (width 0.2) (layer "F.Cu") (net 2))
 (segment (start 123.868838 90.902434) (end 124.128286 90.642986) (width 0.2) (layer "F.Cu") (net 2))
 (segment (start 119.882934 92.15) (end 119.070434 92.9625) (width 0.2) (layer "F.Cu") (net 2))
 (segment (start 124.060916 93.559895) (end 123.760915 93.259894) (width 0.2) (layer "F.Cu") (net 2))
 (segment (start 123.760915 93.259894) (end 123.098416 93.259894) (width 0.2) (layer "F.Cu") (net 2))
 (segment (start 123.098416 95.159894) (end 123.451468 95.159894) (width 0.2) (layer "F.Cu") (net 2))
 (segment (start 121.957934 90.040256) (end 121.642678 89.725) (width 0.2) (layer "F.Cu") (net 2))
 (segment (start 124.060916 94.550446) (end 124.060916 93.559895) (width 0.2) (layer "F.Cu") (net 2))
 (segment (start 122.15 76.35) (end 123 75.5) (width 0.2) (layer "F.Cu") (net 8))
 (segment (start 125.440786 87.931597) (end 125.440786 89.352434) (width 0.2) (layer "F.Cu") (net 8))
 (segment (start 125.638 83.483586) (end 125.033914 82.8795) (width 0.2) (layer "F.Cu") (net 8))
 (segment (start 123.0375 82.2875) (end 123.0375 81.5) (width 0.2) (layer "F.Cu") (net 8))
 (segment (start 125.0375 87.528311) (end 125.0375 85.6175) (width 0.2) (layer "F.Cu") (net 8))
 (segment (start 125.097 85.558) (end 125.638 85.017) (width 0.2) (layer "F.Cu") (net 8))
 (segment (start 123.6295 82.8795) (end 123.0375 82.2875) (width 0.2) (layer "F.Cu") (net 8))
 (segment (start 125.0375 87.528311) (end 125.440786 87.931597) (width 0.2) (layer "F.Cu") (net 8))
 (segment (start 123.0375 79.5) (end 122.15 78.6125) (width 0.2) (layer "F.Cu") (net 8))
 (segment (start 125.033914 82.8795) (end 123.6295 82.8795) (width 0.2) (layer "F.Cu") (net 8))
 (segment (start 123.0375 79.5) (end 123.0375 81.5) (width 0.2) (layer "F.Cu") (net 8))
 (segment (start 125.0375 85.6175) (end 125.097 85.558) (width 0.2) (layer "F.Cu") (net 8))
 (segment (start 125.638 85.017) (end 125.638 83.483586) (width 0.2) (layer "F.Cu") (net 8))
 (segment (start 122.15 78.6125) (end 122.15 76.35) (width 0.2) (layer "F.Cu") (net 8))
 (segment (start 124.613522 92.5) (end 125.373416 93.259894) (width 0.2) (layer "F.Cu") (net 5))
 (segment (start 118 77.75) (end 117.725 77.475) (width 0.2) (layer "F.Cu") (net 5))
 (segment (start 125.5 93.386478) (end 125.373416 93.259894) (width 0.2) (layer "F.Cu") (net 5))
 (segment (start 119.609744 77.75) (end 118 77.75) (width 0.2) (layer "F.Cu") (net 5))
 (segment (start 121.070434 90.75) (end 122.820434 92.5) (width 0.2) (layer "F.Cu") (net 5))
 (segment (start 125.5 94.25) (end 125.5 93.386478) (width 0.2) (layer "F.Cu") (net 5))
 (segment (start 119.750671 80.748998) (end 119.925 80.574669) (width 0.2) (layer "F.Cu") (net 5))
 (segment (start 117.725 75.4875) (end 118.75 74.4625) (width 0.2) (layer "F.Cu") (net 5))
 (segment (start 119.925 80.574669) (end 119.925 78.065256) (width 0.2) (layer "F.Cu") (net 5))
 (segment (start 117.725 77.475) (end 117.725 75.4875) (width 0.2) (layer "F.Cu") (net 5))
 (segment (start 122.820434 92.5) (end 124.613522 92.5) (width 0.2) (layer "F.Cu") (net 5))
 (segment (start 119.925 78.065256) (end 119.609744 77.75) (width 0.2) (layer "F.Cu") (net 5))
 (via (at 125.5 94.25) (size 0.6) (drill 0.3) (layers "F.Cu" "B.Cu") (free yes) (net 5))
 (via (at 119.750671 80.748998) (size 0.6) (drill 0.3) (layers "F.Cu" "B.Cu") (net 5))
 (segment (start 119.750671 80.748998) (end 119.75 80.749669) (width 0.2) (layer "B.Cu") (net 5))
 (segment (start 119.75 88.5) (end 125.5 94.25) (width 0.2) (layer "B.Cu") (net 5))
 (segment (start 119.75 80.749669) (end 119.75 88.5) (width 0.2) (layer "B.Cu") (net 5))
 (segment (start 125.097 83.5795) (end 125.097 83.922) (width 0.2) (layer "F.Cu") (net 23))
 (segment (start 124.797 83.2795) (end 125.097 83.5795) (width 0.2) (layer "F.Cu") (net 23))
 (segment (start 121.057923 83.2795) (end 124.797 83.2795) (width 0.2) (layer "F.Cu") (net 23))
 (segment (start 120.633279 83.704144) (end 121.057923 83.2795) (width 0.2) (layer "F.Cu") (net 23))
 (segment (start 119.330828 80.080828) (end 119.25 80) (width 0.2) (layer "F.Cu") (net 15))
 (segment (start 118.75 81.8) (end 118.75 82.25) (width 0.2) (layer "F.Cu") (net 15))
 (segment (start 118.75 78.7) (end 118.75 81.8) (width 0.2) (layer "F.Cu") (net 15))
 (segment (start 119.253886 80.003886) (end 119.253886 80.080828) (width 0.2) (layer "F.Cu") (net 15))
 (segment (start 118.75 78.7) (end 118.75 79.5) (width 0.2) (layer "F.Cu") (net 15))
 (segment (start 118.75 79.5) (end 119.253886 80.003886) (width 0.2) (layer "F.Cu") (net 15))
 (segment (start 118.75 82.25) (end 118.558279 82.441721) (width 0.2) (layer "F.Cu") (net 15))
 (segment (start 119.253886 80.080828) (end 119.330828 80.080828) (width 0.2) (layer "F.Cu") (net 15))
 (segment (start 118.558279 82.441721) (end 118.558279 83.704144) (width 0.2) (layer "F.Cu") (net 15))
 (via (at 119.253886 80.080828) (size 0.6) (drill 0.3) (layers "F.Cu" "B.Cu") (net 15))
 (segment (start 119.253886 80.080828) (end 119.75 79.584714) (width 0.2) (layer "B.Cu") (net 15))
 (segment (start 119.75 79.584714) (end 119.75 75.75) (width 0.2) (layer "B.Cu") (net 15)))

